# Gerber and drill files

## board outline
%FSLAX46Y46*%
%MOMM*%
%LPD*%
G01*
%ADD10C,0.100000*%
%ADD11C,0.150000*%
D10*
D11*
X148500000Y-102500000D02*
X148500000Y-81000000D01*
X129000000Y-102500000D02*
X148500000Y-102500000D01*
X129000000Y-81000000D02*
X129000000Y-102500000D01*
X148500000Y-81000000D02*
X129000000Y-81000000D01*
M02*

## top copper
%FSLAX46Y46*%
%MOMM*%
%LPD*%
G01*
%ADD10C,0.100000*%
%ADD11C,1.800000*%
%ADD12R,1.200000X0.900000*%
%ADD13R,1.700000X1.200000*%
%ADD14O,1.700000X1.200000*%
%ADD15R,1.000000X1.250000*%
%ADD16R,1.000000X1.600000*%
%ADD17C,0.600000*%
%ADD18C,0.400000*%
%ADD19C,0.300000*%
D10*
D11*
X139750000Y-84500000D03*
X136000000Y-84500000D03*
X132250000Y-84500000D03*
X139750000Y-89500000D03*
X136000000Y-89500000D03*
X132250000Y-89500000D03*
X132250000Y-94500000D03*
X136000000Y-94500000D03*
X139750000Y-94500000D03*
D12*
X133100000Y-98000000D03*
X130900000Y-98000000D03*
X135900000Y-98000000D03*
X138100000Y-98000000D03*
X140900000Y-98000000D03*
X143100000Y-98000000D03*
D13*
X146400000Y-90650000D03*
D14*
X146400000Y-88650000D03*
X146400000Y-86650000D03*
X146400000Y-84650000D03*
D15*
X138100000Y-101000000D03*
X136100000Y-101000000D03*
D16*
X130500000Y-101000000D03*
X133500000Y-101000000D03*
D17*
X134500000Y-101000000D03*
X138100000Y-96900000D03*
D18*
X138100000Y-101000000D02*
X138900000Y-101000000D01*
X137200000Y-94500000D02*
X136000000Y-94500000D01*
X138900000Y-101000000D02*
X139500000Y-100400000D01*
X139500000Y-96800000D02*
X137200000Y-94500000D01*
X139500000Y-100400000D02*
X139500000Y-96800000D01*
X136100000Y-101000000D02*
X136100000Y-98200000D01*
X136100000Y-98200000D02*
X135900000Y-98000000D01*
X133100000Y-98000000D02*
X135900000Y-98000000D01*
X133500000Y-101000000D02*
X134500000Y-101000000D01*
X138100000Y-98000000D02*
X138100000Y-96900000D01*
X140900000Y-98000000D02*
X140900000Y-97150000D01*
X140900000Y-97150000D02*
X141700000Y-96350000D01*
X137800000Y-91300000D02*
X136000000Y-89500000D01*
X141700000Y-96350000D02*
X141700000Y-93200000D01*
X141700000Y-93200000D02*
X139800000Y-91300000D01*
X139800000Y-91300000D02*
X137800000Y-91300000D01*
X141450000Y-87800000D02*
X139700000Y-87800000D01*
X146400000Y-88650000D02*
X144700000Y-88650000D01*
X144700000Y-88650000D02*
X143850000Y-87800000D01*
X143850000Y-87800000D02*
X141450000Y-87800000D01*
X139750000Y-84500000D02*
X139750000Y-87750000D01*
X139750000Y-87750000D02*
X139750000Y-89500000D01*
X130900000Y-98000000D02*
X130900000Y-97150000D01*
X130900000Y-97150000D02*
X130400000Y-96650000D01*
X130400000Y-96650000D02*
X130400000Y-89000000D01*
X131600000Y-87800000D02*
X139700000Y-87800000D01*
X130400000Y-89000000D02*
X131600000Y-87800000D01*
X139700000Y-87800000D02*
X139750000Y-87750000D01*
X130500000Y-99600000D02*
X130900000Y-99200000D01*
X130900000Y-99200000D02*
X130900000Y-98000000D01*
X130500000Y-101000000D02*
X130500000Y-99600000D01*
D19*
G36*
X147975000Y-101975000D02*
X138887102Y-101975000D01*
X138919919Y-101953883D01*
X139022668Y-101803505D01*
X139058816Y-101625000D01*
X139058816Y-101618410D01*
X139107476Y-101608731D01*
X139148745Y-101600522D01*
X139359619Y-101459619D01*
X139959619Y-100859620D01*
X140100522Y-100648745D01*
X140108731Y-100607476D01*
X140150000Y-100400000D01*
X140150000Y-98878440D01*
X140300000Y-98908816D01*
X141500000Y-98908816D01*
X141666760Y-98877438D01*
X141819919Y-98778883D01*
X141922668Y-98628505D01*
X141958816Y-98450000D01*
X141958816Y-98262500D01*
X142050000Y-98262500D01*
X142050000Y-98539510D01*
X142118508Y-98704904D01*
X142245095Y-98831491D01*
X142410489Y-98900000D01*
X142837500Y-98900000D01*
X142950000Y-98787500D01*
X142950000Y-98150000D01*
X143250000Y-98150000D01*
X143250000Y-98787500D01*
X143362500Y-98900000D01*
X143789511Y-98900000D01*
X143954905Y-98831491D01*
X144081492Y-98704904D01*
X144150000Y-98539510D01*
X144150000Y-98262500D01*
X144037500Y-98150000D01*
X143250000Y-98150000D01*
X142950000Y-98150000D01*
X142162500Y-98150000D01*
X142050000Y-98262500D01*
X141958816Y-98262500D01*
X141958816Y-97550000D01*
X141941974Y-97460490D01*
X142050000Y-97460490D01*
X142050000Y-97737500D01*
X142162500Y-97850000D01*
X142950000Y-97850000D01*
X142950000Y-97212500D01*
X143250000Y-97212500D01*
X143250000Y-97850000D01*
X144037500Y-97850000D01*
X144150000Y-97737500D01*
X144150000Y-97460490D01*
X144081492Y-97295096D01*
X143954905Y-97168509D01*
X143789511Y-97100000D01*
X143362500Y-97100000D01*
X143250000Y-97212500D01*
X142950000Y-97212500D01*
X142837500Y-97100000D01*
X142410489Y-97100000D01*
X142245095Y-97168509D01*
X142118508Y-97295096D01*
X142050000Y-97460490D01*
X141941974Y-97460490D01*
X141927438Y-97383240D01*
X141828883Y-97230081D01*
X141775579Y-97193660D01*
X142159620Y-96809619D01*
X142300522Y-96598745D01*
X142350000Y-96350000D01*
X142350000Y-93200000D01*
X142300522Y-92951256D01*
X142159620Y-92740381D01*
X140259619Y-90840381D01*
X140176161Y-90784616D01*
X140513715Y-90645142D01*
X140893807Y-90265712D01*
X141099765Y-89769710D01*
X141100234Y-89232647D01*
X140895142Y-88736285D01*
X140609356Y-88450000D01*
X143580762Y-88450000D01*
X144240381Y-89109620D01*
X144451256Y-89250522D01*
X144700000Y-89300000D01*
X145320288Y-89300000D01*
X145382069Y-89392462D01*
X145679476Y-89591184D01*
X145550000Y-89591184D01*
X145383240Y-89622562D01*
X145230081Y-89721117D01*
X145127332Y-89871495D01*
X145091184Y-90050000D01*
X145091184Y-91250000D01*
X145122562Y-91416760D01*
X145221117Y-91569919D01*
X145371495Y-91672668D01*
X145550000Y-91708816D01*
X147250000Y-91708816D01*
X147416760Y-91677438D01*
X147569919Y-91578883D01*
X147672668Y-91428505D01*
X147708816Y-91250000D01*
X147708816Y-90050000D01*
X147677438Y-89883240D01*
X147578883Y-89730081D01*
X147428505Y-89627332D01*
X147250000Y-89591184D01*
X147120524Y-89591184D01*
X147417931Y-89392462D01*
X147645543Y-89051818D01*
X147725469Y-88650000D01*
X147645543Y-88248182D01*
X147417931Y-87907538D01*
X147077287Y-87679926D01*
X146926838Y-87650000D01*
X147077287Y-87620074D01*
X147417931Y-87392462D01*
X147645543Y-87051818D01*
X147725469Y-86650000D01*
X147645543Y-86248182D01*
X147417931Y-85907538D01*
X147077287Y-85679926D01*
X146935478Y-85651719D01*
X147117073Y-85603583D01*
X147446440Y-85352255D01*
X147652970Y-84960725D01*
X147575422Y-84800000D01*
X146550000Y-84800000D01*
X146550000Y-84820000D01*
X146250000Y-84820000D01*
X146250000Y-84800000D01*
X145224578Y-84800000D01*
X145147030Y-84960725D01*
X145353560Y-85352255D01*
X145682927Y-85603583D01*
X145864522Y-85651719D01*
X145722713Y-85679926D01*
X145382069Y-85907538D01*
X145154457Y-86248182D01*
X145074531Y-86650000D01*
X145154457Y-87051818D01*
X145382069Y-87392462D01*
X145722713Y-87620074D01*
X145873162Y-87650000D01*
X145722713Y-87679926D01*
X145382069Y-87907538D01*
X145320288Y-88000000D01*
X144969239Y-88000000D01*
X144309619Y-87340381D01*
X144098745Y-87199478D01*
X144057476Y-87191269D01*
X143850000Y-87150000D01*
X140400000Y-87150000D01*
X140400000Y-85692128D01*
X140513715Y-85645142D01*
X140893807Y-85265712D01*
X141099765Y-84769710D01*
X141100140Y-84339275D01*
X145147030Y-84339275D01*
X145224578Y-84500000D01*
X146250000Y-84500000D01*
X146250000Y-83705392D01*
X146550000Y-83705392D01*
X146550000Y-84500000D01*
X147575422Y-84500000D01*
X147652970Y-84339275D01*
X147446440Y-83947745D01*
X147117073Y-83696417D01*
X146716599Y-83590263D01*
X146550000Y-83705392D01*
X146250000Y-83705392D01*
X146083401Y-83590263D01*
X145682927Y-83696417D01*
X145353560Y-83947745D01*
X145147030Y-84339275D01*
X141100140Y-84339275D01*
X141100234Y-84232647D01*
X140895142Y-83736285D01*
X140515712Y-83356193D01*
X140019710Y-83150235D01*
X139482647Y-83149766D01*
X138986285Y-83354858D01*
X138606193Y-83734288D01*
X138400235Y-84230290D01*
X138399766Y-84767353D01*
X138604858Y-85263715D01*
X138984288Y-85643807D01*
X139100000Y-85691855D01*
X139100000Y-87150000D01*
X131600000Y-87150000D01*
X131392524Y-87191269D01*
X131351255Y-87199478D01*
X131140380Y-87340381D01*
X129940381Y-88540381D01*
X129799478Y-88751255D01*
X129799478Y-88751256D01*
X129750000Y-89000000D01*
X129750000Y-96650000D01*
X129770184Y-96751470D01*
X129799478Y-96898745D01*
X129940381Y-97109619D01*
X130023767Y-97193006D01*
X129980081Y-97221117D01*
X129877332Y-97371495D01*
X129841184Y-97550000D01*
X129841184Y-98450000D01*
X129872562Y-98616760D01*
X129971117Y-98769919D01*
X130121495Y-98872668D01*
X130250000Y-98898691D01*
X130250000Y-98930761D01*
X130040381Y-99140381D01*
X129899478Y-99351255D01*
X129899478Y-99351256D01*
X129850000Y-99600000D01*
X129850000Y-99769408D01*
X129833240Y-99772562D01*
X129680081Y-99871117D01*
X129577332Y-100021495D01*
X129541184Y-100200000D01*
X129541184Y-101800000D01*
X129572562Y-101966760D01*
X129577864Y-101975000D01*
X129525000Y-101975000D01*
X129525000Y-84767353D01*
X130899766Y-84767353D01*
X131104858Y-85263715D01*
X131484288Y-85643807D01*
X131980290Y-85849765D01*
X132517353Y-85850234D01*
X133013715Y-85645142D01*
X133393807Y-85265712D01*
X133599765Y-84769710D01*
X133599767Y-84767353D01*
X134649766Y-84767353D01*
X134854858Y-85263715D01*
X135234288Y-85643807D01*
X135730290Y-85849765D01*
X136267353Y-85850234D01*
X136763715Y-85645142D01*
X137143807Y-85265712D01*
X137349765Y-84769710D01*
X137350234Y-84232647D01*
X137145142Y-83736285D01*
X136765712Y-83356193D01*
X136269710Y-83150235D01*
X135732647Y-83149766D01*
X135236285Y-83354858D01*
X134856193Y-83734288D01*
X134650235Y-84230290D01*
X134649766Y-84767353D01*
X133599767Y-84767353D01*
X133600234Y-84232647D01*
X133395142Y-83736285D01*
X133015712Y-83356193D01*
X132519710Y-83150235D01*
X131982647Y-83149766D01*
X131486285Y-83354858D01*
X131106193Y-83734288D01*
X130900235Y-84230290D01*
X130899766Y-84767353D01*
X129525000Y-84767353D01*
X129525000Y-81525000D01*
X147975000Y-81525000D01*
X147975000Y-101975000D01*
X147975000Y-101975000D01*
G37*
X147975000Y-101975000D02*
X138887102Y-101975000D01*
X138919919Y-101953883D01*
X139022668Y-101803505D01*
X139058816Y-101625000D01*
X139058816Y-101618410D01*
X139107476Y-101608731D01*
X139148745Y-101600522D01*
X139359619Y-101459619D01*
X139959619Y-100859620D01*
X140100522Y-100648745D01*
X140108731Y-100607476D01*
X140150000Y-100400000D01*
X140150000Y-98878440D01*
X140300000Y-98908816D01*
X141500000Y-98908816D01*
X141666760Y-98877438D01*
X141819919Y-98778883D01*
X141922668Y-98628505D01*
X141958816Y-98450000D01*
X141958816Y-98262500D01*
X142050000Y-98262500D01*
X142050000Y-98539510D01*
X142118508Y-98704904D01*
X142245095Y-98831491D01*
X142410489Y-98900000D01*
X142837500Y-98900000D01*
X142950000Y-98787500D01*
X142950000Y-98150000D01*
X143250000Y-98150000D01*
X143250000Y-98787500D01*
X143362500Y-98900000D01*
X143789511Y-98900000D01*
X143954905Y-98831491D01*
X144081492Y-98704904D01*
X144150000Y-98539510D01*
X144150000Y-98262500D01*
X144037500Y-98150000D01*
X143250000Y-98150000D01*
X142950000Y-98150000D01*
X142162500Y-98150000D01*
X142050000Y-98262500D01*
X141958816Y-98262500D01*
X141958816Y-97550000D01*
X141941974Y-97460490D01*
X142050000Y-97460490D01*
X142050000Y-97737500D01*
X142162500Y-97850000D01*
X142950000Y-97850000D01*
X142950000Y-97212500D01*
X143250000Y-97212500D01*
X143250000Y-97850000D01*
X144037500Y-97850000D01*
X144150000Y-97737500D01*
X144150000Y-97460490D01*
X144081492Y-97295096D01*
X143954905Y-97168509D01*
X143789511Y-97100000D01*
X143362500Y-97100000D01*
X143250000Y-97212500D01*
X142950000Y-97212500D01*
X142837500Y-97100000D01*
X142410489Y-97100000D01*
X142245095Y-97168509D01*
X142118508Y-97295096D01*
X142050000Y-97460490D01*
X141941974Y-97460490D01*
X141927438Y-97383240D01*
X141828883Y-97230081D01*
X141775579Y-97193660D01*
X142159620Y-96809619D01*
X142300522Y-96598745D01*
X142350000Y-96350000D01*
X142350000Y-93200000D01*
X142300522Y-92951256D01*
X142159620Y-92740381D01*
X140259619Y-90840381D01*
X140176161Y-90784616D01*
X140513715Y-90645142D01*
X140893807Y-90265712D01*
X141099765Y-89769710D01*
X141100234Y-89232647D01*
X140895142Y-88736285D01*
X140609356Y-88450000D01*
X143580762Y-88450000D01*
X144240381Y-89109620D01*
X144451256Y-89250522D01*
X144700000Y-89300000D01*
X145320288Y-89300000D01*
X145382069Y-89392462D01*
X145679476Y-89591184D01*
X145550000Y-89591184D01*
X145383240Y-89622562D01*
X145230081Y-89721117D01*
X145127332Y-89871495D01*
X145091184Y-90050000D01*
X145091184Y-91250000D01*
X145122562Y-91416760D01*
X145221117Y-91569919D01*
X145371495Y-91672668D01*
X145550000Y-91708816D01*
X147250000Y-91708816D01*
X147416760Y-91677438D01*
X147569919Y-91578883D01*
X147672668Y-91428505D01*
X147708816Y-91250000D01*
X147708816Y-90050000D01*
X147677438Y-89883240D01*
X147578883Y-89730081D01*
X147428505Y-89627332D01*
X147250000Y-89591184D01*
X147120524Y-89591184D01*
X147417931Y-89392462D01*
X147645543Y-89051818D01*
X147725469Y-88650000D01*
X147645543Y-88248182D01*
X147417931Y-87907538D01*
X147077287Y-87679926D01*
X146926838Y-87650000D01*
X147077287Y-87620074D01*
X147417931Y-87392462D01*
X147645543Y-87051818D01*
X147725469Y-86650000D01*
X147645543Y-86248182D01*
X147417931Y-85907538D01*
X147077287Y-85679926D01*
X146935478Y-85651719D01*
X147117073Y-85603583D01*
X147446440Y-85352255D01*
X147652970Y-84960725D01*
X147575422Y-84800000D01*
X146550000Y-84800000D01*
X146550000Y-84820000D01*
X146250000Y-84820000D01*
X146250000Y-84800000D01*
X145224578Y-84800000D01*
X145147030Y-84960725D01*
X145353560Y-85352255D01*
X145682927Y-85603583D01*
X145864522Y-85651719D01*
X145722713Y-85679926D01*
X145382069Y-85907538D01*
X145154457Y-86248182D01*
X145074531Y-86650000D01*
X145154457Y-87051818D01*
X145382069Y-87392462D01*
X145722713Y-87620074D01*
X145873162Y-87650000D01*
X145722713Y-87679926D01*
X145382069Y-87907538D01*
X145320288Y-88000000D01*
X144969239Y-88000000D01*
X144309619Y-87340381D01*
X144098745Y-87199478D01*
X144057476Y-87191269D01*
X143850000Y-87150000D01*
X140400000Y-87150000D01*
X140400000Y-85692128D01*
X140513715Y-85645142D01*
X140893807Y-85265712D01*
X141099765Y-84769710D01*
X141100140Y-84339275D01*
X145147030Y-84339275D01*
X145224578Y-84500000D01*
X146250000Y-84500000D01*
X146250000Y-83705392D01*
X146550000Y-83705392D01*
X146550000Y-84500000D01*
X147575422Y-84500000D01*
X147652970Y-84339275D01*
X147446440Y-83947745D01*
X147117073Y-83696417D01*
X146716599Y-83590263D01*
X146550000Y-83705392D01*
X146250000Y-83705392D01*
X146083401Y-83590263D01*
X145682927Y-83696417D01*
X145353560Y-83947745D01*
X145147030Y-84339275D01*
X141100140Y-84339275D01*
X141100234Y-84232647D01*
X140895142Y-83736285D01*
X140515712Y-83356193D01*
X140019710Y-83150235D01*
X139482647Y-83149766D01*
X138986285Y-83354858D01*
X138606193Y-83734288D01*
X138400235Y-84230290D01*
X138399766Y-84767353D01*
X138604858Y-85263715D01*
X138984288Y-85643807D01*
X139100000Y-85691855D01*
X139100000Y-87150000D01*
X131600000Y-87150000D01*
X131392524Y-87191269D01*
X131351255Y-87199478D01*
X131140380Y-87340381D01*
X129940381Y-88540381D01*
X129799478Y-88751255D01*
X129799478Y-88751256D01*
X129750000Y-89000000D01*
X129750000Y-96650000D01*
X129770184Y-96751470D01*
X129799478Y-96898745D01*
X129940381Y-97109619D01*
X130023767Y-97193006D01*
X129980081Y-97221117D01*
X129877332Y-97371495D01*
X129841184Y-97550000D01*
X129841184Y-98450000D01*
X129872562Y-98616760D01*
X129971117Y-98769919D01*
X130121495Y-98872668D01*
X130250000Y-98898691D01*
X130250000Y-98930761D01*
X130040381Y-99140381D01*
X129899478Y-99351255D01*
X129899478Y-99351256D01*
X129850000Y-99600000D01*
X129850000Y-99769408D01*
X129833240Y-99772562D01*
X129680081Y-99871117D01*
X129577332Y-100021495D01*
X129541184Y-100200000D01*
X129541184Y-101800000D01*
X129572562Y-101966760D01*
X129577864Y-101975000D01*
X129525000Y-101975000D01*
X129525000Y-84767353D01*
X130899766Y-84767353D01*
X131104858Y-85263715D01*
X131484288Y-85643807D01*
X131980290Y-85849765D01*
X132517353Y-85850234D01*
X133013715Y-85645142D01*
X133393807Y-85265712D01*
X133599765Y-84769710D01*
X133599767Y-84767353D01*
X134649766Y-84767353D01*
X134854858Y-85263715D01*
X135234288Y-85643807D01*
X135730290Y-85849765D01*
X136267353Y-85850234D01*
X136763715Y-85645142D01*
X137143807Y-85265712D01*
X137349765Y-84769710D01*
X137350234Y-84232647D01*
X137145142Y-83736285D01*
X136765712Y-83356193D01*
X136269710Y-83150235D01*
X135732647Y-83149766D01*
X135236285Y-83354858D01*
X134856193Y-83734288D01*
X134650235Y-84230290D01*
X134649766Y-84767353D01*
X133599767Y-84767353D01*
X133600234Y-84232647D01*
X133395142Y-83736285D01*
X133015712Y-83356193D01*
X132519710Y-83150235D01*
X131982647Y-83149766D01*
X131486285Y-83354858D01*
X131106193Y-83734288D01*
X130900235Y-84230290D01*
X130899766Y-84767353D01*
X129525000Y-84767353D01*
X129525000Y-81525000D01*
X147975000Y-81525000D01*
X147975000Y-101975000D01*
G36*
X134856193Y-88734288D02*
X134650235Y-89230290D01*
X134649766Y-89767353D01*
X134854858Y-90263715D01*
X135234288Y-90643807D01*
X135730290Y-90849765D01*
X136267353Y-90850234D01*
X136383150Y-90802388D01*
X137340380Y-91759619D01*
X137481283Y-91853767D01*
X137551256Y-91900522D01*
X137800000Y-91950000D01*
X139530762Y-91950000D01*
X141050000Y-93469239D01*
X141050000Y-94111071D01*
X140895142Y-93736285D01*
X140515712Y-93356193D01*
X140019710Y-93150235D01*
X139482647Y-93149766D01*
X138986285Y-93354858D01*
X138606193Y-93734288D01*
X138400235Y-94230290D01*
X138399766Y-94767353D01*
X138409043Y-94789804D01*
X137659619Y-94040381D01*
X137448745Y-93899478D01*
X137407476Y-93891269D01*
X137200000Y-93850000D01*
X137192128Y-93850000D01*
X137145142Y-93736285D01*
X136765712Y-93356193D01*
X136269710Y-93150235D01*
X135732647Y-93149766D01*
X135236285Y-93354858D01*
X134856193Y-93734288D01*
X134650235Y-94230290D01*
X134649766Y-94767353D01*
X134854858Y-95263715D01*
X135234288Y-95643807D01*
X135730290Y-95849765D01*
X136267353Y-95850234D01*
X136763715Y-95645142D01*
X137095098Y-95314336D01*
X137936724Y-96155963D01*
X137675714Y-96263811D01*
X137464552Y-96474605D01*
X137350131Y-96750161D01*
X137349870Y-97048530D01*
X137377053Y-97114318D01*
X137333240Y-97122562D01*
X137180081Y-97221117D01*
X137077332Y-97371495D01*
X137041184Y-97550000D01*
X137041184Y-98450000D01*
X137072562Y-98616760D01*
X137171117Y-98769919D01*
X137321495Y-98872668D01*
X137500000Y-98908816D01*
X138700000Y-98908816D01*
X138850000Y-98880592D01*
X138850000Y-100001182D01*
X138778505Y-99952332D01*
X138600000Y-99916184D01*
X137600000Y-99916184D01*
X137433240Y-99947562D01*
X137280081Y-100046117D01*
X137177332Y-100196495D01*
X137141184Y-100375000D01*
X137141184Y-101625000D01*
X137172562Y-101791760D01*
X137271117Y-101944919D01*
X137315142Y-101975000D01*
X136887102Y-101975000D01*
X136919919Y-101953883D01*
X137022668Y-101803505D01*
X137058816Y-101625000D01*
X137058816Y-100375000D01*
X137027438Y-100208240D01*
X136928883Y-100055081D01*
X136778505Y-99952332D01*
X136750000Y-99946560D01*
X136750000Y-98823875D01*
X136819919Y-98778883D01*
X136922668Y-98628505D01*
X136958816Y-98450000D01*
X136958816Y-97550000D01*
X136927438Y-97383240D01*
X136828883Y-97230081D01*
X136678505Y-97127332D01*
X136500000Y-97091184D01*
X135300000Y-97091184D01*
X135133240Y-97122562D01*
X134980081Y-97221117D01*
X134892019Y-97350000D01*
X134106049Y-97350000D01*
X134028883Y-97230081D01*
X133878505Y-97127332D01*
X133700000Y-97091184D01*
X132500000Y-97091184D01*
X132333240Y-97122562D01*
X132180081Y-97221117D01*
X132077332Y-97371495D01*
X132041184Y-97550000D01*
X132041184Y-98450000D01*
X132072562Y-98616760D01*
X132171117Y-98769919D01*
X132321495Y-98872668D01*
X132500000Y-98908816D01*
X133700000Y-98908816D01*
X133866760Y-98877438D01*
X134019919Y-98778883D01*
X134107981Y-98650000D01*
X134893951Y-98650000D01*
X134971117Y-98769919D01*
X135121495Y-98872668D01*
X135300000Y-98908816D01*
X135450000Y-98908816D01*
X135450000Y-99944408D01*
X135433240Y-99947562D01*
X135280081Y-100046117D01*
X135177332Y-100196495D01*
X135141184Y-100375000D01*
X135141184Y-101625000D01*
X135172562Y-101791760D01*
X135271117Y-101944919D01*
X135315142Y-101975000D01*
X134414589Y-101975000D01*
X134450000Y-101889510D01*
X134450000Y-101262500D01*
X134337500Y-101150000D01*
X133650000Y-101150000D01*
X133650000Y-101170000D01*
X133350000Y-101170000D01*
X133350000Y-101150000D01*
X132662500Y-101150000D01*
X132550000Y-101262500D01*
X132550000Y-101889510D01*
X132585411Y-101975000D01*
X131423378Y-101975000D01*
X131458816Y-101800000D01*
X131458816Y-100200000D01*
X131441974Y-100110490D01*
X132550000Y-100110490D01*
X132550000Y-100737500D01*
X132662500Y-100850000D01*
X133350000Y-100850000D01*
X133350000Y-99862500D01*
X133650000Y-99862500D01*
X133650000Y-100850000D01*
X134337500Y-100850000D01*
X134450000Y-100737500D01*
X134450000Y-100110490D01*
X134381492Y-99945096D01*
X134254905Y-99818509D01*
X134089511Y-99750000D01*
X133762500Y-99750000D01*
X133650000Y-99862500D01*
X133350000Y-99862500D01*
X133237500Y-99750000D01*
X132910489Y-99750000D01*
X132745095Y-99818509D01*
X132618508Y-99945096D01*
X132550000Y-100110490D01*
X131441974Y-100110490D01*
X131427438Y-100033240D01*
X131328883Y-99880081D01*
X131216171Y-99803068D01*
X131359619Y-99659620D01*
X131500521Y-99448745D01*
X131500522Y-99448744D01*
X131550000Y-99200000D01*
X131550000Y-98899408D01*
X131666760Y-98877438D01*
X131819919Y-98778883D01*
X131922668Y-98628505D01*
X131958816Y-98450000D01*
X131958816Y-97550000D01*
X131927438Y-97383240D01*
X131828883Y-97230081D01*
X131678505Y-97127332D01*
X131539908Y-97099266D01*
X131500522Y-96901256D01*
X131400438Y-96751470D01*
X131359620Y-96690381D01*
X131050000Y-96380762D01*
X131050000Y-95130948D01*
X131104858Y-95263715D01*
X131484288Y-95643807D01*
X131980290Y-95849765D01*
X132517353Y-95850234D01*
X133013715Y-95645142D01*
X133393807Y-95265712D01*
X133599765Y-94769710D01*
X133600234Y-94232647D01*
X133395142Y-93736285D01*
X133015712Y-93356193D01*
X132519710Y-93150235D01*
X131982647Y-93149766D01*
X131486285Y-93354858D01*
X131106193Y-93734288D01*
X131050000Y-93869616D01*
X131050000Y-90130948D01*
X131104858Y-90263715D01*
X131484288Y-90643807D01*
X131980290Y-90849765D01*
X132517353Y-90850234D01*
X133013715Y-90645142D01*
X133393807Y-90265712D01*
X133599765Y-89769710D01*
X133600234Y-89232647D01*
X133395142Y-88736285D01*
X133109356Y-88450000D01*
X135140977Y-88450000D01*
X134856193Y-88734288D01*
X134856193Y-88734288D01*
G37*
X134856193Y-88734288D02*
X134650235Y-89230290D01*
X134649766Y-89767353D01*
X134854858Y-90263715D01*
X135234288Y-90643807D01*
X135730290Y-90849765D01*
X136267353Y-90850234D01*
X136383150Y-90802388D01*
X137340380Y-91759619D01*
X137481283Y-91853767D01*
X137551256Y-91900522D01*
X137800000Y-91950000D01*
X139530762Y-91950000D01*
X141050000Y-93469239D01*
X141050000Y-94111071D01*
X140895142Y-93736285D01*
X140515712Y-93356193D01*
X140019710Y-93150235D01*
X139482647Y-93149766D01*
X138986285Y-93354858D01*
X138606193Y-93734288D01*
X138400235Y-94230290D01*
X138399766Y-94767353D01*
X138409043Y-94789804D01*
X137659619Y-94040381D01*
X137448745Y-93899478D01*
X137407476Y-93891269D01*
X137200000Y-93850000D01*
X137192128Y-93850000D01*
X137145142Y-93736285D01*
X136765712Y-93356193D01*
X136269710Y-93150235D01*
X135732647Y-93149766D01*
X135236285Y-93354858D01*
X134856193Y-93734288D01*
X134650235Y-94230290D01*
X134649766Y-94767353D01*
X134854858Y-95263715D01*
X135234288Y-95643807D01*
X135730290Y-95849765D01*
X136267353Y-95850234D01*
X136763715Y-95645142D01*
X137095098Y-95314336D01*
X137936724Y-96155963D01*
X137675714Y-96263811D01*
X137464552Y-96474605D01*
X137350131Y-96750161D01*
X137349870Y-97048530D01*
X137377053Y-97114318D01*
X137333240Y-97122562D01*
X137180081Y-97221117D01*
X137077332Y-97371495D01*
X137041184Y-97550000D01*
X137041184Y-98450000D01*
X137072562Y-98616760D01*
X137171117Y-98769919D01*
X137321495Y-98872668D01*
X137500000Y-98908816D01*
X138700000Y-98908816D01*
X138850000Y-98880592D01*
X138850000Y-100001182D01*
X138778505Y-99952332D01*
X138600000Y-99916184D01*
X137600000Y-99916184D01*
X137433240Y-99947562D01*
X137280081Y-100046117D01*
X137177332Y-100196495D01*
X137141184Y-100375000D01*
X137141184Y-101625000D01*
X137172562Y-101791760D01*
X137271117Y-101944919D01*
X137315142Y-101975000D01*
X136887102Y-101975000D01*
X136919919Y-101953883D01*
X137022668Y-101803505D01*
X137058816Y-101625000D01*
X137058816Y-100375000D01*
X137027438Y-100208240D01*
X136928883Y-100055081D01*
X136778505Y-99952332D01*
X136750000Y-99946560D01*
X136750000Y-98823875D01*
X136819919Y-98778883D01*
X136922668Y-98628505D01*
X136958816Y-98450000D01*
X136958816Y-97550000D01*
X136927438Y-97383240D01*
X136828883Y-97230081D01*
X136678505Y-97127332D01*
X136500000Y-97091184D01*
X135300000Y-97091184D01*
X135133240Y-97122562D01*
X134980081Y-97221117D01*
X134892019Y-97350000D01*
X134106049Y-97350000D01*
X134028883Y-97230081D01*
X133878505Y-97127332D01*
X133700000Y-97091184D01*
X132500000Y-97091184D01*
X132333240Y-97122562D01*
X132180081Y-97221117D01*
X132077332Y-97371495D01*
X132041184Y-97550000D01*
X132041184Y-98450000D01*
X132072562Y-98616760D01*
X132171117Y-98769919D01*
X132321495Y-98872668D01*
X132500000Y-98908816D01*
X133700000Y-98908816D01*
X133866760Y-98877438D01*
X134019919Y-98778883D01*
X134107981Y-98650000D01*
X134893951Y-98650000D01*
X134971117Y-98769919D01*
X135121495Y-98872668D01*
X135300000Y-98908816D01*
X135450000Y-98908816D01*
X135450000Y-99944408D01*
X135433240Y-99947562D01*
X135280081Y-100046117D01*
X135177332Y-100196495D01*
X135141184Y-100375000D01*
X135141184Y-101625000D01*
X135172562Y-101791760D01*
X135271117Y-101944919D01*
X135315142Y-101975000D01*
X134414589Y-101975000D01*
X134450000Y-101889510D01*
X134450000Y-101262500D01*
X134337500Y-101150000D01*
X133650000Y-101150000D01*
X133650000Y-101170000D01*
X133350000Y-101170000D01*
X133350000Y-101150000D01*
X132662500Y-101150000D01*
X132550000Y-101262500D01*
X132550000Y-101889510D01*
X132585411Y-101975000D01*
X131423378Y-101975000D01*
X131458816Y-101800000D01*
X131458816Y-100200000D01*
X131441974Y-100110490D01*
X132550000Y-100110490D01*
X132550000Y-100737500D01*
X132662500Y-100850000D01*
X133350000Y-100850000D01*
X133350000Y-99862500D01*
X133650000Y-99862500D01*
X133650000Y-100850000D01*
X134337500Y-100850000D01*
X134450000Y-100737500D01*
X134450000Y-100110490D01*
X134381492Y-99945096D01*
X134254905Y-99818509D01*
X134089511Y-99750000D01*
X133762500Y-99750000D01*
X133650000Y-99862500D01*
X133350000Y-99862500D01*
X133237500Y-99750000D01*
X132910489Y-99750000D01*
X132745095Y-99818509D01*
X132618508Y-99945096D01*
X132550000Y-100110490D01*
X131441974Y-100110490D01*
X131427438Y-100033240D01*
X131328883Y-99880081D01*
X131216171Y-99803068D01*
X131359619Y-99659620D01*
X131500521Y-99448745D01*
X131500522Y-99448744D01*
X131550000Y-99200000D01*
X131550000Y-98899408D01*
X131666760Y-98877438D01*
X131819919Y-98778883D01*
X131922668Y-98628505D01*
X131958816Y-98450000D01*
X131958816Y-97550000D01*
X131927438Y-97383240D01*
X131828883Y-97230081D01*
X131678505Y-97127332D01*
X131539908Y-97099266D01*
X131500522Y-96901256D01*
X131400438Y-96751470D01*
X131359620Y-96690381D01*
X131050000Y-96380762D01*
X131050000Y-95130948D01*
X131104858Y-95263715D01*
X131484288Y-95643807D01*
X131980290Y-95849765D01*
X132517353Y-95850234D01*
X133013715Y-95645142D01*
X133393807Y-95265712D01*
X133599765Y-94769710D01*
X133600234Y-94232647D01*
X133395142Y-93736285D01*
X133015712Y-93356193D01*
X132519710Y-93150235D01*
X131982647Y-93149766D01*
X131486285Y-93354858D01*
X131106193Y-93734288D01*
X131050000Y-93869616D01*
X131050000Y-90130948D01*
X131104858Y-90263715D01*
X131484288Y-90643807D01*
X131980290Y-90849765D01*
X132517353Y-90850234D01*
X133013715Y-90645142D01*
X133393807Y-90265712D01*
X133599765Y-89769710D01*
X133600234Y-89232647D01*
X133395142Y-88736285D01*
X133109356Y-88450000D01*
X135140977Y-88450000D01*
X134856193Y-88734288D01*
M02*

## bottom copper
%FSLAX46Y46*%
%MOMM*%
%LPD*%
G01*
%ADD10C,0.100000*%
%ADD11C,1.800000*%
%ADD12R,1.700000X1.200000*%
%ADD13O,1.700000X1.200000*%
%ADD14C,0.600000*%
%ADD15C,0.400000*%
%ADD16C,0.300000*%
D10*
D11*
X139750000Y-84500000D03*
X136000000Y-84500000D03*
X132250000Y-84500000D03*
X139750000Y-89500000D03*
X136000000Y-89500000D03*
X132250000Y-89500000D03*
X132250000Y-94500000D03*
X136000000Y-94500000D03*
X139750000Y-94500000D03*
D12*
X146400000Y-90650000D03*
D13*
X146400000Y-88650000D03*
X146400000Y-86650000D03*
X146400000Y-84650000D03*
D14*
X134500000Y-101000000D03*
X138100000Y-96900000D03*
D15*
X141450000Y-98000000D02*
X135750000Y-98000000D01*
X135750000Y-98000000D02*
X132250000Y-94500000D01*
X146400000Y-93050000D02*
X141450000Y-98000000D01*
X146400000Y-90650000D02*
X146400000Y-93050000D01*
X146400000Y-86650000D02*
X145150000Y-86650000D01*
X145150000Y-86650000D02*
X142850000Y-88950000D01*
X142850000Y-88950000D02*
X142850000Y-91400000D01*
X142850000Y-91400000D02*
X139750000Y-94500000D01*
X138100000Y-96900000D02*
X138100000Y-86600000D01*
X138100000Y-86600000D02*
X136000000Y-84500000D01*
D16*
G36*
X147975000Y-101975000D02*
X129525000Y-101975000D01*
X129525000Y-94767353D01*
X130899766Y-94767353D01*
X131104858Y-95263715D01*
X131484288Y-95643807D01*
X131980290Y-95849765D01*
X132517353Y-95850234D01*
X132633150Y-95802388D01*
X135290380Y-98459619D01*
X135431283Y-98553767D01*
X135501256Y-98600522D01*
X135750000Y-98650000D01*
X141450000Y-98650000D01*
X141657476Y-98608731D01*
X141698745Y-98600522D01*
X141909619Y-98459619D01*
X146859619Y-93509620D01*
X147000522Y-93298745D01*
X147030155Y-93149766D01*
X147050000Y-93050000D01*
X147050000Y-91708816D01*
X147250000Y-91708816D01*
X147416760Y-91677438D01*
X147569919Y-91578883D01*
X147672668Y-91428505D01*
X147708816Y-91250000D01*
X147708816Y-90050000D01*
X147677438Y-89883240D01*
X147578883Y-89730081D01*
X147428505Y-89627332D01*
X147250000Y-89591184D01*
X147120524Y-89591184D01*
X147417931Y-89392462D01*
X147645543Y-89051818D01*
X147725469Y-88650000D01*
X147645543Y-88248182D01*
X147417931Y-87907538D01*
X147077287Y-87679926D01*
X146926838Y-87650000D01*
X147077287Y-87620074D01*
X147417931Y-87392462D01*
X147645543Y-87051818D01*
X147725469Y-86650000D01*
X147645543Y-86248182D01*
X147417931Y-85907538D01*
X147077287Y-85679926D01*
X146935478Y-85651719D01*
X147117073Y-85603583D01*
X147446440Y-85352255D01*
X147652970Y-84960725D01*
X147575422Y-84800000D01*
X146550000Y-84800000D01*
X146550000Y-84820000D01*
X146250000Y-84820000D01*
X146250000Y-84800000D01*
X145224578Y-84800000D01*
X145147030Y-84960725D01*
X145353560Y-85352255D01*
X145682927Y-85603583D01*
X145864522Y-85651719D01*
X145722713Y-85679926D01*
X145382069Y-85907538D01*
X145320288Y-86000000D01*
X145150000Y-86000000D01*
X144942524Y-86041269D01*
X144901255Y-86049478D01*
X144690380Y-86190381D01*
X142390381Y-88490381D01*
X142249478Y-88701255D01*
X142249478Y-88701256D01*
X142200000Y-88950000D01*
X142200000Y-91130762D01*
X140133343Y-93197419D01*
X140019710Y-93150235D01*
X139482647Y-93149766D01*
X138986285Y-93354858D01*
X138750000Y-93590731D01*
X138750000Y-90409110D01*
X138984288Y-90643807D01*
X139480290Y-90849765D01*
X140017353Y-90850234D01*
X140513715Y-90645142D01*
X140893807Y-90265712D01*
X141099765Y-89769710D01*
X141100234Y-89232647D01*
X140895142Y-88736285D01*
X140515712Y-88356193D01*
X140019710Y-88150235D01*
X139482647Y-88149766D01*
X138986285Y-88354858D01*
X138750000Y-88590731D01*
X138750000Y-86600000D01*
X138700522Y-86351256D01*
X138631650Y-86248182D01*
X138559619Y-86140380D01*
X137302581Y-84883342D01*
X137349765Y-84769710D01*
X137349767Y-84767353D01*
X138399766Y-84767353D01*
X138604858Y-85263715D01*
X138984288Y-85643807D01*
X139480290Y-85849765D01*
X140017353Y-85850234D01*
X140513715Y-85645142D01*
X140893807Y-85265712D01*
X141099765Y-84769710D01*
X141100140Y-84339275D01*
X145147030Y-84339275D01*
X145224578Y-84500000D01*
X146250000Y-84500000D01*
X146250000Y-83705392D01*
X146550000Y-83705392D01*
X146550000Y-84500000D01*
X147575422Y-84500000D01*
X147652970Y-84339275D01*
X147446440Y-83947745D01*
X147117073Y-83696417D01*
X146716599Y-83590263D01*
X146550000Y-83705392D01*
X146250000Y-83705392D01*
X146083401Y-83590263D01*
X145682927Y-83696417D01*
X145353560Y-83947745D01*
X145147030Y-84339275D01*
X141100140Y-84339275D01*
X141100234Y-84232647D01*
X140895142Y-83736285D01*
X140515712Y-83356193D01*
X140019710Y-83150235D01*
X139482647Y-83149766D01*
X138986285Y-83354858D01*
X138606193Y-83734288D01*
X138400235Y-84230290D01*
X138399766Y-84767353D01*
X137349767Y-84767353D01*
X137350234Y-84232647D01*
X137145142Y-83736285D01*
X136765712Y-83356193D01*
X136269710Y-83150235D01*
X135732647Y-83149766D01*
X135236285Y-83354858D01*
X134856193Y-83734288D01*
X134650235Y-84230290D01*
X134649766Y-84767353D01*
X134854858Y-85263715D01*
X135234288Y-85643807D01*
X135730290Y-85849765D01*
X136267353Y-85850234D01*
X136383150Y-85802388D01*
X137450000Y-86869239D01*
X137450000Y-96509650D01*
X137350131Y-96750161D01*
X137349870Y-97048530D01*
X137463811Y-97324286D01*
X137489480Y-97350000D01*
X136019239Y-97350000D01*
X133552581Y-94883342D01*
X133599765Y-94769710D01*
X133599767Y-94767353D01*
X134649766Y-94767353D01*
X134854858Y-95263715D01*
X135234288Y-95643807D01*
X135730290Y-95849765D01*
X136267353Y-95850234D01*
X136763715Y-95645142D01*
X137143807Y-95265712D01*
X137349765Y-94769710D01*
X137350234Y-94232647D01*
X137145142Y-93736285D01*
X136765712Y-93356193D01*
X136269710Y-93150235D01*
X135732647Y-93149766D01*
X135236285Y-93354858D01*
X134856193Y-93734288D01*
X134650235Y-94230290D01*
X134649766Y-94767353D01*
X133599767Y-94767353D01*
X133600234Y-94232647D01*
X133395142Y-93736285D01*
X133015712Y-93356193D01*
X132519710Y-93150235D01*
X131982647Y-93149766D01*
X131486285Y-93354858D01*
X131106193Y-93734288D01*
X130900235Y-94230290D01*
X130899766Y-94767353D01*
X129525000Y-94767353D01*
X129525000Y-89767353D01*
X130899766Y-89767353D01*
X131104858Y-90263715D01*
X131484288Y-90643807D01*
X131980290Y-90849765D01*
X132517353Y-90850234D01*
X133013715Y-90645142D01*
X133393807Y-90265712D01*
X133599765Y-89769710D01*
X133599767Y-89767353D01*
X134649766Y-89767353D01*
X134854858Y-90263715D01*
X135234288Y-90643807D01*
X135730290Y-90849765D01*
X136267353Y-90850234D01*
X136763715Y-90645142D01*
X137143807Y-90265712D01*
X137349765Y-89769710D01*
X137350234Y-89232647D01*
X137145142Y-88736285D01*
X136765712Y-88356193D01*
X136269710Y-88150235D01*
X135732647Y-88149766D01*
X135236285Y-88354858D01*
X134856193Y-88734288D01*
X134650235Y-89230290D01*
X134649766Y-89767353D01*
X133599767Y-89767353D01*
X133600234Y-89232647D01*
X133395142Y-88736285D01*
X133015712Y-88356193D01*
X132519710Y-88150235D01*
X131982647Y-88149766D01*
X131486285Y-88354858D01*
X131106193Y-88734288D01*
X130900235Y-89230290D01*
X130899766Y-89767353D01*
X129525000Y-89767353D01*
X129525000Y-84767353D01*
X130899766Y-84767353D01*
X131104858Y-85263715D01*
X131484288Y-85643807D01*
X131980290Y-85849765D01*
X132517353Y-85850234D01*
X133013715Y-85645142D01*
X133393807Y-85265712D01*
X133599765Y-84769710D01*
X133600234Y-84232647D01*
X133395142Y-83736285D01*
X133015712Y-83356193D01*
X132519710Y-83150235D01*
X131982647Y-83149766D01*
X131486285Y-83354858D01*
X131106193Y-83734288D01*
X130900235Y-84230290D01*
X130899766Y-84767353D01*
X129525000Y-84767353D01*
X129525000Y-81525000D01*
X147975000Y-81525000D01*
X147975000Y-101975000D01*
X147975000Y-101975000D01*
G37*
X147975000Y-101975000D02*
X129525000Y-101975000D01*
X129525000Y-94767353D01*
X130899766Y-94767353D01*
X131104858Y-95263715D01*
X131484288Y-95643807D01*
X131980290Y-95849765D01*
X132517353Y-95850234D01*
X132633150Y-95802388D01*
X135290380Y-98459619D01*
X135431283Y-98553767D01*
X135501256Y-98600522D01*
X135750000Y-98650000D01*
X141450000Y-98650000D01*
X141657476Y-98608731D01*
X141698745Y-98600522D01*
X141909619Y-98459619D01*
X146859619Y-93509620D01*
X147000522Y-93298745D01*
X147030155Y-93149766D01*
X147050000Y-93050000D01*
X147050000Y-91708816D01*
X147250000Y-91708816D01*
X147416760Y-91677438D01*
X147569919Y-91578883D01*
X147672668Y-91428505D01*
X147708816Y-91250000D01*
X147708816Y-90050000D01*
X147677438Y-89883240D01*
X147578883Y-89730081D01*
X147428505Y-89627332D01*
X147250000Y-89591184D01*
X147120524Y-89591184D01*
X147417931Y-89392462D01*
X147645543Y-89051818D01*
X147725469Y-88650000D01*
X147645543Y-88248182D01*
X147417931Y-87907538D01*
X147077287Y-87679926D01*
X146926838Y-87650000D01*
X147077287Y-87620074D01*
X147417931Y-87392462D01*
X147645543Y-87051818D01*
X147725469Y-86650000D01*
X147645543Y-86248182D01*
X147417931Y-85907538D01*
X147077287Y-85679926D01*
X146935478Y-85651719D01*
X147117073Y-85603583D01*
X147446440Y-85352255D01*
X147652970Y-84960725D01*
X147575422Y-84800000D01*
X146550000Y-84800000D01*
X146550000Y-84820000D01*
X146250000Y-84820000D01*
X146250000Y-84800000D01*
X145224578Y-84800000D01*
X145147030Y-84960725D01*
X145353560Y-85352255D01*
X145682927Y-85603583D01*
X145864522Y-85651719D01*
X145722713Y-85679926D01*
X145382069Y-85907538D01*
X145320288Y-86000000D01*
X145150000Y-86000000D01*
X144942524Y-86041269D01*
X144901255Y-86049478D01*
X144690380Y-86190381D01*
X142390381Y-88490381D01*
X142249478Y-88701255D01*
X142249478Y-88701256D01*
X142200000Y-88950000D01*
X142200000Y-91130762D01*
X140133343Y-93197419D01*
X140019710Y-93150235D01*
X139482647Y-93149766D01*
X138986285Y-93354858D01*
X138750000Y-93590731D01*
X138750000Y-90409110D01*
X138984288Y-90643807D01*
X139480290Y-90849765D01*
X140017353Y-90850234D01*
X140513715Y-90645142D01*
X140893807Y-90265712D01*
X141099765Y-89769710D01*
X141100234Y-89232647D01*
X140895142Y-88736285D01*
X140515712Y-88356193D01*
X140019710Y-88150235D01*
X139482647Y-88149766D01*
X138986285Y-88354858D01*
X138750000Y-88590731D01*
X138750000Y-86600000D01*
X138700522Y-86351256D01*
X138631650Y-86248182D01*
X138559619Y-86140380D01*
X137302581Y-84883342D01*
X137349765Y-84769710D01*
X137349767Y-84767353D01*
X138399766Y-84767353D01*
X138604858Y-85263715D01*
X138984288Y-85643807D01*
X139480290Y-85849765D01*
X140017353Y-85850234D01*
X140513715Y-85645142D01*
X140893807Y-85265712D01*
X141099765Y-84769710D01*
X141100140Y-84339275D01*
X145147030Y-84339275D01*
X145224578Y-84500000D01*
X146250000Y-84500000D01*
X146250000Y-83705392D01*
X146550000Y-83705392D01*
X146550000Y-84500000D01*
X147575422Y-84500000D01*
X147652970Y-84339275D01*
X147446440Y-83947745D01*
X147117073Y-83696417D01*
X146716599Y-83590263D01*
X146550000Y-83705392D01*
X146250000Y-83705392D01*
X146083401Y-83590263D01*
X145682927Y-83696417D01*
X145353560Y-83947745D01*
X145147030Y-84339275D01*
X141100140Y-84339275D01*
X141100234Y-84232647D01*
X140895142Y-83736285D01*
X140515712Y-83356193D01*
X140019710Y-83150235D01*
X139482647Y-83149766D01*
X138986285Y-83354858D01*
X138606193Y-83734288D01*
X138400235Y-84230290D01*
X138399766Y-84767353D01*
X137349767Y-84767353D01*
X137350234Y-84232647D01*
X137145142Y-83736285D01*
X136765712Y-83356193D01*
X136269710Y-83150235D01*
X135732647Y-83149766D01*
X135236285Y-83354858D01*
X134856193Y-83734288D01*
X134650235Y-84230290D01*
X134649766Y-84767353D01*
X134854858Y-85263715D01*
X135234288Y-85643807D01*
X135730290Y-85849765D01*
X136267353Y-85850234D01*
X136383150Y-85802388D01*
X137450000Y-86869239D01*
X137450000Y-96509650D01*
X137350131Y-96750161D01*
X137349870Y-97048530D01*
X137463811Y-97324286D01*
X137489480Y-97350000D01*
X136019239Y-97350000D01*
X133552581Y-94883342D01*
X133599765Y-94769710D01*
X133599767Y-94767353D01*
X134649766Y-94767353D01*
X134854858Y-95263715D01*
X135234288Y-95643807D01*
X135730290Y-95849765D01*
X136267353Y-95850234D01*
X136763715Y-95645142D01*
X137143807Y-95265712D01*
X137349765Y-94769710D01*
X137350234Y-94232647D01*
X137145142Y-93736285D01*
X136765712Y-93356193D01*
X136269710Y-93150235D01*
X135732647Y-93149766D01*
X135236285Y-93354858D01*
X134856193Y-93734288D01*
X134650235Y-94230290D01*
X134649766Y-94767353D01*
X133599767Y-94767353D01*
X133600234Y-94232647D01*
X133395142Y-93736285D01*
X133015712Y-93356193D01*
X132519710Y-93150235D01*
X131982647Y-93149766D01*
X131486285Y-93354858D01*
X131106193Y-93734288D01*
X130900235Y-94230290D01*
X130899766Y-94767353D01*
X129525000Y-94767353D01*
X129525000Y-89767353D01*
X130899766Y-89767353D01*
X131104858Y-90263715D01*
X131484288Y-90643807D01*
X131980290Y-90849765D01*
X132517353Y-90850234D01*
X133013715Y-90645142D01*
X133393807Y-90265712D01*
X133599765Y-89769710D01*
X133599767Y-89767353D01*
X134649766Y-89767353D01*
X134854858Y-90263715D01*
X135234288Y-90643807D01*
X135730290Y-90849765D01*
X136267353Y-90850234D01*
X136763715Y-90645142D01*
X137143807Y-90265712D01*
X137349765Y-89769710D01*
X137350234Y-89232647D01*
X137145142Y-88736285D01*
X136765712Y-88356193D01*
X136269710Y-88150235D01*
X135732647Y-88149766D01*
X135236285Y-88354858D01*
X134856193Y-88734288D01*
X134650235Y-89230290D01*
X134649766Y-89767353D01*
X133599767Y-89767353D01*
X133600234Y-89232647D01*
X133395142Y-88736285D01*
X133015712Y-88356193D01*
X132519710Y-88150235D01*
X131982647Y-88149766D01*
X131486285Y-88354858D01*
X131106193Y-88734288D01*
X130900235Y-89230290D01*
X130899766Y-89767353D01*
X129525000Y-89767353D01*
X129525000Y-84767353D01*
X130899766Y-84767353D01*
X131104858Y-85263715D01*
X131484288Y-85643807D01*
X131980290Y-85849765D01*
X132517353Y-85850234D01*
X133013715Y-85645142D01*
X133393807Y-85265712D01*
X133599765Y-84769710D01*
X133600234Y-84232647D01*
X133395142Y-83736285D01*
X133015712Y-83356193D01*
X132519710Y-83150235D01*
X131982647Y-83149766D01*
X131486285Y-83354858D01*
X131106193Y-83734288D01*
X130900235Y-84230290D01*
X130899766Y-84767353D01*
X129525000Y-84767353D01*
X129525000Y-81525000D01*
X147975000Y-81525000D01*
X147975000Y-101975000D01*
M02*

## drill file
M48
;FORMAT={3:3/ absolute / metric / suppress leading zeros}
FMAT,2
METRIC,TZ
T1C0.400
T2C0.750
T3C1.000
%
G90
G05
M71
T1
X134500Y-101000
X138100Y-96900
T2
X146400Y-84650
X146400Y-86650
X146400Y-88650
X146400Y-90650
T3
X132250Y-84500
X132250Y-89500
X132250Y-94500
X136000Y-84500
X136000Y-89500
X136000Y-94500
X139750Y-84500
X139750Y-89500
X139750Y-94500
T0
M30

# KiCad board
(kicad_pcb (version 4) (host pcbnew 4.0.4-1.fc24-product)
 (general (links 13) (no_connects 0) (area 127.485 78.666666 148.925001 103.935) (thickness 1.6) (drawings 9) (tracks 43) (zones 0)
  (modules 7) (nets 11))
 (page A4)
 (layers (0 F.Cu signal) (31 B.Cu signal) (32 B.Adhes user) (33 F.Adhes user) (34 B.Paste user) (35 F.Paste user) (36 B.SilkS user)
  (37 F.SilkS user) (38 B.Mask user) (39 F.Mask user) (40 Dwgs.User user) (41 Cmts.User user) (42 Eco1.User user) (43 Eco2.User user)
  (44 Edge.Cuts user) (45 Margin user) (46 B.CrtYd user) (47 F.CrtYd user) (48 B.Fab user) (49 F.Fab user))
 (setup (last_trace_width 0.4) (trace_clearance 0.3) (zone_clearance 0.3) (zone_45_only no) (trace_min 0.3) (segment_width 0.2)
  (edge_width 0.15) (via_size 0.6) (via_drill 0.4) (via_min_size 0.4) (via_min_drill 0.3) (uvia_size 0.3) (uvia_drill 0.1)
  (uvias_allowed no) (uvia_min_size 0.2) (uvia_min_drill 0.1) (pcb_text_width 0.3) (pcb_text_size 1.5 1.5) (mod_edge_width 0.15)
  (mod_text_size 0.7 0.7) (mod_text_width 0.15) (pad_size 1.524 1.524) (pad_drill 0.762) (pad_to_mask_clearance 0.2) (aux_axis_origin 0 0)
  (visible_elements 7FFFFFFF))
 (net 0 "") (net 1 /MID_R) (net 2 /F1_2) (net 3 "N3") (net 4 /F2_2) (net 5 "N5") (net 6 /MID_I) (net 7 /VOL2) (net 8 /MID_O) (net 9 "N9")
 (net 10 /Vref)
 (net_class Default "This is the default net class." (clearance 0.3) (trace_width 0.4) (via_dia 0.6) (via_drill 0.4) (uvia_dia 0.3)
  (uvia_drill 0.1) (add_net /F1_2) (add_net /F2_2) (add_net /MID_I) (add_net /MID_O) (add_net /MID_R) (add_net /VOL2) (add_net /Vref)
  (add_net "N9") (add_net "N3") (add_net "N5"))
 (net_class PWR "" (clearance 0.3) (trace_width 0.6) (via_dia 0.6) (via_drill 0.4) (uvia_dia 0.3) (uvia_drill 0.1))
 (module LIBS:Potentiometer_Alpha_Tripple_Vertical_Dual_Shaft (layer B.Cu) (at 132.25 84.5 90)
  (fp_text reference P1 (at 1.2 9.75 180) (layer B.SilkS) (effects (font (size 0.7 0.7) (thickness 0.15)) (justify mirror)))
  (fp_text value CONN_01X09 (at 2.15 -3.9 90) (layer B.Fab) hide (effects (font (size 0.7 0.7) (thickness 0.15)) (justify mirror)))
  (pad 3 thru_hole circle (at 0 7.5 90) (size 1.8 1.8) (drill 1) (layers *.Cu *.Mask) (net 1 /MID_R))
  (pad 2 thru_hole circle (at 0 3.75 90) (size 1.8 1.8) (drill 1) (layers *.Cu *.Mask) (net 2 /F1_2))
  (pad 1 thru_hole circle (at 0 0 90) (size 1.8 1.8) (drill 1) (layers *.Cu *.Mask) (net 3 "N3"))
  (pad 6 thru_hole circle (at -5 7.5 90) (size 1.8 1.8) (drill 1) (layers *.Cu *.Mask) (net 1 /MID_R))
  (pad 5 thru_hole circle (at -5 3.75 90) (size 1.8 1.8) (drill 1) (layers *.Cu *.Mask) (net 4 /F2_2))
  (pad 4 thru_hole circle (at -5 0 90) (size 1.8 1.8) (drill 1) (layers *.Cu *.Mask) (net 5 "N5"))
  (pad 7 thru_hole circle (at -10 0 90) (size 1.8 1.8) (drill 1) (layers *.Cu *.Mask) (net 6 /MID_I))
  (pad 8 thru_hole circle (at -10 3.75 90) (size 1.8 1.8) (drill 1) (layers *.Cu *.Mask) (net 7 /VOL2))
  (pad 9 thru_hole circle (at -10 7.5 90) (size 1.8 1.8) (drill 1) (layers *.Cu *.Mask) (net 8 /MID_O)))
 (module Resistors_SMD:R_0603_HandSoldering (layer F.Cu) (at 132 98 180)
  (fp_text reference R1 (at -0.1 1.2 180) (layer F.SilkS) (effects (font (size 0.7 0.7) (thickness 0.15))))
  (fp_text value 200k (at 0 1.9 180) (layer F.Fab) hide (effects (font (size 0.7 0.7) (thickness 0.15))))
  (pad 1 smd rect (at -1.1 0 180) (size 1.2 0.9) (layers F.Cu F.Paste F.Mask) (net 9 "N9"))
  (pad 2 smd rect (at 1.1 0 180) (size 1.2 0.9) (layers F.Cu F.Paste F.Mask) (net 1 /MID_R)))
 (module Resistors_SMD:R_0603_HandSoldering (layer F.Cu) (at 137 98)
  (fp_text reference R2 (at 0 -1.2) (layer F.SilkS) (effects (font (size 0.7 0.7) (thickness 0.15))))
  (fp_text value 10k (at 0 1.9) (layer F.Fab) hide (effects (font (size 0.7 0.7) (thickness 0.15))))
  (pad 1 smd rect (at -1.1 0) (size 1.2 0.9) (layers F.Cu F.Paste F.Mask) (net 9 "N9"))
  (pad 2 smd rect (at 1.1 0) (size 1.2 0.9) (layers F.Cu F.Paste F.Mask) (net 2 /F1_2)))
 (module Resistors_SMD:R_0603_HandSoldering (layer F.Cu) (at 142 98)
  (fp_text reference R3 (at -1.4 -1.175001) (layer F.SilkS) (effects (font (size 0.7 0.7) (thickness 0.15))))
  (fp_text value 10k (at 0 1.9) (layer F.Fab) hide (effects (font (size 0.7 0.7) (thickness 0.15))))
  (pad 1 smd rect (at -1.1 0) (size 1.2 0.9) (layers F.Cu F.Paste F.Mask) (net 4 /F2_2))
  (pad 2 smd rect (at 1.1 0) (size 1.2 0.9) (layers F.Cu F.Paste F.Mask) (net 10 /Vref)))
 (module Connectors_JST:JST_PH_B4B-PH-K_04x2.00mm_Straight (layer B.Cu) (at 146.4 90.65 90)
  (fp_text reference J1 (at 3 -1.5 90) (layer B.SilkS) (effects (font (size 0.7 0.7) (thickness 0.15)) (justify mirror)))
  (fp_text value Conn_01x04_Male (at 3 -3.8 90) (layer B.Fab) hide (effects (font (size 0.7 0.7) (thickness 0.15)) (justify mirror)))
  (pad 1 thru_hole rect (at 0 0 90) (size 1.2 1.7) (drill 0.75) (layers *.Cu *.Mask) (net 6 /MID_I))
  (pad 2 thru_hole oval (at 2 0 90) (size 1.2 1.7) (drill 0.75) (layers *.Cu *.Mask) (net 1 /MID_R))
  (pad 3 thru_hole oval (at 4 0 90) (size 1.2 1.7) (drill 0.75) (layers *.Cu *.Mask) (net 8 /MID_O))
  (pad 4 thru_hole oval (at 6 0 90) (size 1.2 1.7) (drill 0.75) (layers *.Cu *.Mask) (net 10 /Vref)))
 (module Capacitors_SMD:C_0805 (layer F.Cu) (at 137.1 101 180)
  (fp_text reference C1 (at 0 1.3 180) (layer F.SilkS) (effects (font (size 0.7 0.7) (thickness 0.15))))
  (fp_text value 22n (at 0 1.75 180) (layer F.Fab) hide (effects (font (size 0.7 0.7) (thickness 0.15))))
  (pad 1 smd rect (at -1 0 180) (size 1 1.25) (layers F.Cu F.Paste F.Mask) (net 7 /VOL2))
  (pad 2 smd rect (at 1 0 180) (size 1 1.25) (layers F.Cu F.Paste F.Mask) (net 9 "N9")))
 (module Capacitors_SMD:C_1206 (layer F.Cu) (at 132 101)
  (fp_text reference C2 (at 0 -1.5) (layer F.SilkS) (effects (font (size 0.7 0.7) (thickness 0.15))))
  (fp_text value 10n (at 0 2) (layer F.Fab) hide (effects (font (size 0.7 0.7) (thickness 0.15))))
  (pad 1 smd rect (at -1.5 0) (size 1 1.6) (layers F.Cu F.Paste F.Mask) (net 1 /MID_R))
  (pad 2 smd rect (at 1.5 0) (size 1 1.6) (layers F.Cu F.Paste F.Mask) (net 10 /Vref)))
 (gr_line (start 148.5 102.5) (end 148.5 81) (layer Edge.Cuts) (width 0.15))
 (gr_line (start 129 102.5) (end 148.5 102.5) (layer Edge.Cuts) (width 0.15))
 (gr_line (start 129 81) (end 129 102.5) (layer Edge.Cuts) (width 0.15))
 (gr_line (start 148.5 81) (end 129 81) (layer Edge.Cuts) (width 0.15))
 (segment (start 138.1 101) (end 138.9 101) (width 0.4) (layer F.Cu) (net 7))
 (segment (start 137.2 94.5) (end 136 94.5) (width 0.4) (layer F.Cu) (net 7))
 (segment (start 138.9 101) (end 139.5 100.4) (width 0.4) (layer F.Cu) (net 7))
 (segment (start 139.5 96.8) (end 137.2 94.5) (width 0.4) (layer F.Cu) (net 7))
 (segment (start 139.5 100.4) (end 139.5 96.8) (width 0.4) (layer F.Cu) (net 7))
 (segment (start 136.1 101) (end 136.1 98.2) (width 0.4) (layer F.Cu) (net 9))
 (segment (start 136.1 98.2) (end 135.9 98) (width 0.4) (layer F.Cu) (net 9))
 (segment (start 133.1 98) (end 135.9 98) (width 0.4) (layer F.Cu) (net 9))
 (segment (start 133.5 101) (end 134.5 101) (width 0.4) (layer F.Cu) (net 10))
 (via (at 134.5 101) (size 0.6) (drill 0.4) (layers F.Cu B.Cu) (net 10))
 (segment (start 141.45 98) (end 135.75 98) (width 0.4) (layer B.Cu) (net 6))
 (segment (start 135.75 98) (end 132.25 94.5) (width 0.4) (layer B.Cu) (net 6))
 (segment (start 146.4 93.05) (end 141.45 98) (width 0.4) (layer B.Cu) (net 6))
 (segment (start 146.4 90.65) (end 146.4 93.05) (width 0.4) (layer B.Cu) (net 6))
 (segment (start 146.4 86.65) (end 145.15 86.65) (width 0.4) (layer B.Cu) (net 8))
 (segment (start 145.15 86.65) (end 142.85 88.95) (width 0.4) (layer B.Cu) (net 8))
 (segment (start 142.85 88.95) (end 142.85 91.4) (width 0.4) (layer B.Cu) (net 8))
 (segment (start 142.85 91.4) (end 139.75 94.5) (width 0.4) (layer B.Cu) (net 8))
 (segment (start 138.1 96.9) (end 138.1 86.6) (width 0.4) (layer B.Cu) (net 2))
 (segment (start 138.1 86.6) (end 136 84.5) (width 0.4) (layer B.Cu) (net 2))
 (segment (start 138.1 98) (end 138.1 96.9) (width 0.4) (layer F.Cu) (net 2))
 (via (at 138.1 96.9) (size 0.6) (drill 0.4) (layers F.Cu B.Cu) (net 2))
 (segment (start 140.9 98) (end 140.9 97.15) (width 0.4) (layer F.Cu) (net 4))
 (segment (start 140.9 97.15) (end 141.7 96.35) (width 0.4) (layer F.Cu) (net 4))
 (segment (start 137.8 91.3) (end 136 89.5) (width 0.4) (layer F.Cu) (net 4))
 (segment (start 141.7 96.35) (end 141.7 93.2) (width 0.4) (layer F.Cu) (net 4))
 (segment (start 141.7 93.2) (end 139.8 91.3) (width 0.4) (layer F.Cu) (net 4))
 (segment (start 139.8 91.3) (end 137.8 91.3) (width 0.4) (layer F.Cu) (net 4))
 (segment (start 141.45 87.8) (end 139.7 87.8) (width 0.4) (layer F.Cu) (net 1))
 (segment (start 146.4 88.65) (end 144.7 88.65) (width 0.4) (layer F.Cu) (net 1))
 (segment (start 144.7 88.65) (end 143.85 87.8) (width 0.4) (layer F.Cu) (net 1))
 (segment (start 143.85 87.8) (end 141.45 87.8) (width 0.4) (layer F.Cu) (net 1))
 (segment (start 139.75 84.5) (end 139.75 87.75) (width 0.4) (layer F.Cu) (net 1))
 (segment (start 139.75 87.75) (end 139.75 89.5) (width 0.4) (layer F.Cu) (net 1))
 (segment (start 130.9 98) (end 130.9 97.15) (width 0.4) (layer F.Cu) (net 1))
 (segment (start 130.9 97.15) (end 130.4 96.65) (width 0.4) (layer F.Cu) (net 1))
 (segment (start 130.4 96.65) (end 130.4 89) (width 0.4) (layer F.Cu) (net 1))
 (segment (start 131.6 87.8) (end 139.7 87.8) (width 0.4) (layer F.Cu) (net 1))
 (segment (start 130.4 89) (end 131.6 87.8) (width 0.4) (layer F.Cu) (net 1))
 (segment (start 139.7 87.8) (end 139.75 87.75) (width 0.4) (layer F.Cu) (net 1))
 (segment (start 130.5 99.6) (end 130.9 99.2) (width 0.4) (layer F.Cu) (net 1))
 (segment (start 130.9 99.2) (end 130.9 98) (width 0.4) (layer F.Cu) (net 1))
 (segment (start 130.5 101) (end 130.5 99.6) (width 0.4) (layer F.Cu) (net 1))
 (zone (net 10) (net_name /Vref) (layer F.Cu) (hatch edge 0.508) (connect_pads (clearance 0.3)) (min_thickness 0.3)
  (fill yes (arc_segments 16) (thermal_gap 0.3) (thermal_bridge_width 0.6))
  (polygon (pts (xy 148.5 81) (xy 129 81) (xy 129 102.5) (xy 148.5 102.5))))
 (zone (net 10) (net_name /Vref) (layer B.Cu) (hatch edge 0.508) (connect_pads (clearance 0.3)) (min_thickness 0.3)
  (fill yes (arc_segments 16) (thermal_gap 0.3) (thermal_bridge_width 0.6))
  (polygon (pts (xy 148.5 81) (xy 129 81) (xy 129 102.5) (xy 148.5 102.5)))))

